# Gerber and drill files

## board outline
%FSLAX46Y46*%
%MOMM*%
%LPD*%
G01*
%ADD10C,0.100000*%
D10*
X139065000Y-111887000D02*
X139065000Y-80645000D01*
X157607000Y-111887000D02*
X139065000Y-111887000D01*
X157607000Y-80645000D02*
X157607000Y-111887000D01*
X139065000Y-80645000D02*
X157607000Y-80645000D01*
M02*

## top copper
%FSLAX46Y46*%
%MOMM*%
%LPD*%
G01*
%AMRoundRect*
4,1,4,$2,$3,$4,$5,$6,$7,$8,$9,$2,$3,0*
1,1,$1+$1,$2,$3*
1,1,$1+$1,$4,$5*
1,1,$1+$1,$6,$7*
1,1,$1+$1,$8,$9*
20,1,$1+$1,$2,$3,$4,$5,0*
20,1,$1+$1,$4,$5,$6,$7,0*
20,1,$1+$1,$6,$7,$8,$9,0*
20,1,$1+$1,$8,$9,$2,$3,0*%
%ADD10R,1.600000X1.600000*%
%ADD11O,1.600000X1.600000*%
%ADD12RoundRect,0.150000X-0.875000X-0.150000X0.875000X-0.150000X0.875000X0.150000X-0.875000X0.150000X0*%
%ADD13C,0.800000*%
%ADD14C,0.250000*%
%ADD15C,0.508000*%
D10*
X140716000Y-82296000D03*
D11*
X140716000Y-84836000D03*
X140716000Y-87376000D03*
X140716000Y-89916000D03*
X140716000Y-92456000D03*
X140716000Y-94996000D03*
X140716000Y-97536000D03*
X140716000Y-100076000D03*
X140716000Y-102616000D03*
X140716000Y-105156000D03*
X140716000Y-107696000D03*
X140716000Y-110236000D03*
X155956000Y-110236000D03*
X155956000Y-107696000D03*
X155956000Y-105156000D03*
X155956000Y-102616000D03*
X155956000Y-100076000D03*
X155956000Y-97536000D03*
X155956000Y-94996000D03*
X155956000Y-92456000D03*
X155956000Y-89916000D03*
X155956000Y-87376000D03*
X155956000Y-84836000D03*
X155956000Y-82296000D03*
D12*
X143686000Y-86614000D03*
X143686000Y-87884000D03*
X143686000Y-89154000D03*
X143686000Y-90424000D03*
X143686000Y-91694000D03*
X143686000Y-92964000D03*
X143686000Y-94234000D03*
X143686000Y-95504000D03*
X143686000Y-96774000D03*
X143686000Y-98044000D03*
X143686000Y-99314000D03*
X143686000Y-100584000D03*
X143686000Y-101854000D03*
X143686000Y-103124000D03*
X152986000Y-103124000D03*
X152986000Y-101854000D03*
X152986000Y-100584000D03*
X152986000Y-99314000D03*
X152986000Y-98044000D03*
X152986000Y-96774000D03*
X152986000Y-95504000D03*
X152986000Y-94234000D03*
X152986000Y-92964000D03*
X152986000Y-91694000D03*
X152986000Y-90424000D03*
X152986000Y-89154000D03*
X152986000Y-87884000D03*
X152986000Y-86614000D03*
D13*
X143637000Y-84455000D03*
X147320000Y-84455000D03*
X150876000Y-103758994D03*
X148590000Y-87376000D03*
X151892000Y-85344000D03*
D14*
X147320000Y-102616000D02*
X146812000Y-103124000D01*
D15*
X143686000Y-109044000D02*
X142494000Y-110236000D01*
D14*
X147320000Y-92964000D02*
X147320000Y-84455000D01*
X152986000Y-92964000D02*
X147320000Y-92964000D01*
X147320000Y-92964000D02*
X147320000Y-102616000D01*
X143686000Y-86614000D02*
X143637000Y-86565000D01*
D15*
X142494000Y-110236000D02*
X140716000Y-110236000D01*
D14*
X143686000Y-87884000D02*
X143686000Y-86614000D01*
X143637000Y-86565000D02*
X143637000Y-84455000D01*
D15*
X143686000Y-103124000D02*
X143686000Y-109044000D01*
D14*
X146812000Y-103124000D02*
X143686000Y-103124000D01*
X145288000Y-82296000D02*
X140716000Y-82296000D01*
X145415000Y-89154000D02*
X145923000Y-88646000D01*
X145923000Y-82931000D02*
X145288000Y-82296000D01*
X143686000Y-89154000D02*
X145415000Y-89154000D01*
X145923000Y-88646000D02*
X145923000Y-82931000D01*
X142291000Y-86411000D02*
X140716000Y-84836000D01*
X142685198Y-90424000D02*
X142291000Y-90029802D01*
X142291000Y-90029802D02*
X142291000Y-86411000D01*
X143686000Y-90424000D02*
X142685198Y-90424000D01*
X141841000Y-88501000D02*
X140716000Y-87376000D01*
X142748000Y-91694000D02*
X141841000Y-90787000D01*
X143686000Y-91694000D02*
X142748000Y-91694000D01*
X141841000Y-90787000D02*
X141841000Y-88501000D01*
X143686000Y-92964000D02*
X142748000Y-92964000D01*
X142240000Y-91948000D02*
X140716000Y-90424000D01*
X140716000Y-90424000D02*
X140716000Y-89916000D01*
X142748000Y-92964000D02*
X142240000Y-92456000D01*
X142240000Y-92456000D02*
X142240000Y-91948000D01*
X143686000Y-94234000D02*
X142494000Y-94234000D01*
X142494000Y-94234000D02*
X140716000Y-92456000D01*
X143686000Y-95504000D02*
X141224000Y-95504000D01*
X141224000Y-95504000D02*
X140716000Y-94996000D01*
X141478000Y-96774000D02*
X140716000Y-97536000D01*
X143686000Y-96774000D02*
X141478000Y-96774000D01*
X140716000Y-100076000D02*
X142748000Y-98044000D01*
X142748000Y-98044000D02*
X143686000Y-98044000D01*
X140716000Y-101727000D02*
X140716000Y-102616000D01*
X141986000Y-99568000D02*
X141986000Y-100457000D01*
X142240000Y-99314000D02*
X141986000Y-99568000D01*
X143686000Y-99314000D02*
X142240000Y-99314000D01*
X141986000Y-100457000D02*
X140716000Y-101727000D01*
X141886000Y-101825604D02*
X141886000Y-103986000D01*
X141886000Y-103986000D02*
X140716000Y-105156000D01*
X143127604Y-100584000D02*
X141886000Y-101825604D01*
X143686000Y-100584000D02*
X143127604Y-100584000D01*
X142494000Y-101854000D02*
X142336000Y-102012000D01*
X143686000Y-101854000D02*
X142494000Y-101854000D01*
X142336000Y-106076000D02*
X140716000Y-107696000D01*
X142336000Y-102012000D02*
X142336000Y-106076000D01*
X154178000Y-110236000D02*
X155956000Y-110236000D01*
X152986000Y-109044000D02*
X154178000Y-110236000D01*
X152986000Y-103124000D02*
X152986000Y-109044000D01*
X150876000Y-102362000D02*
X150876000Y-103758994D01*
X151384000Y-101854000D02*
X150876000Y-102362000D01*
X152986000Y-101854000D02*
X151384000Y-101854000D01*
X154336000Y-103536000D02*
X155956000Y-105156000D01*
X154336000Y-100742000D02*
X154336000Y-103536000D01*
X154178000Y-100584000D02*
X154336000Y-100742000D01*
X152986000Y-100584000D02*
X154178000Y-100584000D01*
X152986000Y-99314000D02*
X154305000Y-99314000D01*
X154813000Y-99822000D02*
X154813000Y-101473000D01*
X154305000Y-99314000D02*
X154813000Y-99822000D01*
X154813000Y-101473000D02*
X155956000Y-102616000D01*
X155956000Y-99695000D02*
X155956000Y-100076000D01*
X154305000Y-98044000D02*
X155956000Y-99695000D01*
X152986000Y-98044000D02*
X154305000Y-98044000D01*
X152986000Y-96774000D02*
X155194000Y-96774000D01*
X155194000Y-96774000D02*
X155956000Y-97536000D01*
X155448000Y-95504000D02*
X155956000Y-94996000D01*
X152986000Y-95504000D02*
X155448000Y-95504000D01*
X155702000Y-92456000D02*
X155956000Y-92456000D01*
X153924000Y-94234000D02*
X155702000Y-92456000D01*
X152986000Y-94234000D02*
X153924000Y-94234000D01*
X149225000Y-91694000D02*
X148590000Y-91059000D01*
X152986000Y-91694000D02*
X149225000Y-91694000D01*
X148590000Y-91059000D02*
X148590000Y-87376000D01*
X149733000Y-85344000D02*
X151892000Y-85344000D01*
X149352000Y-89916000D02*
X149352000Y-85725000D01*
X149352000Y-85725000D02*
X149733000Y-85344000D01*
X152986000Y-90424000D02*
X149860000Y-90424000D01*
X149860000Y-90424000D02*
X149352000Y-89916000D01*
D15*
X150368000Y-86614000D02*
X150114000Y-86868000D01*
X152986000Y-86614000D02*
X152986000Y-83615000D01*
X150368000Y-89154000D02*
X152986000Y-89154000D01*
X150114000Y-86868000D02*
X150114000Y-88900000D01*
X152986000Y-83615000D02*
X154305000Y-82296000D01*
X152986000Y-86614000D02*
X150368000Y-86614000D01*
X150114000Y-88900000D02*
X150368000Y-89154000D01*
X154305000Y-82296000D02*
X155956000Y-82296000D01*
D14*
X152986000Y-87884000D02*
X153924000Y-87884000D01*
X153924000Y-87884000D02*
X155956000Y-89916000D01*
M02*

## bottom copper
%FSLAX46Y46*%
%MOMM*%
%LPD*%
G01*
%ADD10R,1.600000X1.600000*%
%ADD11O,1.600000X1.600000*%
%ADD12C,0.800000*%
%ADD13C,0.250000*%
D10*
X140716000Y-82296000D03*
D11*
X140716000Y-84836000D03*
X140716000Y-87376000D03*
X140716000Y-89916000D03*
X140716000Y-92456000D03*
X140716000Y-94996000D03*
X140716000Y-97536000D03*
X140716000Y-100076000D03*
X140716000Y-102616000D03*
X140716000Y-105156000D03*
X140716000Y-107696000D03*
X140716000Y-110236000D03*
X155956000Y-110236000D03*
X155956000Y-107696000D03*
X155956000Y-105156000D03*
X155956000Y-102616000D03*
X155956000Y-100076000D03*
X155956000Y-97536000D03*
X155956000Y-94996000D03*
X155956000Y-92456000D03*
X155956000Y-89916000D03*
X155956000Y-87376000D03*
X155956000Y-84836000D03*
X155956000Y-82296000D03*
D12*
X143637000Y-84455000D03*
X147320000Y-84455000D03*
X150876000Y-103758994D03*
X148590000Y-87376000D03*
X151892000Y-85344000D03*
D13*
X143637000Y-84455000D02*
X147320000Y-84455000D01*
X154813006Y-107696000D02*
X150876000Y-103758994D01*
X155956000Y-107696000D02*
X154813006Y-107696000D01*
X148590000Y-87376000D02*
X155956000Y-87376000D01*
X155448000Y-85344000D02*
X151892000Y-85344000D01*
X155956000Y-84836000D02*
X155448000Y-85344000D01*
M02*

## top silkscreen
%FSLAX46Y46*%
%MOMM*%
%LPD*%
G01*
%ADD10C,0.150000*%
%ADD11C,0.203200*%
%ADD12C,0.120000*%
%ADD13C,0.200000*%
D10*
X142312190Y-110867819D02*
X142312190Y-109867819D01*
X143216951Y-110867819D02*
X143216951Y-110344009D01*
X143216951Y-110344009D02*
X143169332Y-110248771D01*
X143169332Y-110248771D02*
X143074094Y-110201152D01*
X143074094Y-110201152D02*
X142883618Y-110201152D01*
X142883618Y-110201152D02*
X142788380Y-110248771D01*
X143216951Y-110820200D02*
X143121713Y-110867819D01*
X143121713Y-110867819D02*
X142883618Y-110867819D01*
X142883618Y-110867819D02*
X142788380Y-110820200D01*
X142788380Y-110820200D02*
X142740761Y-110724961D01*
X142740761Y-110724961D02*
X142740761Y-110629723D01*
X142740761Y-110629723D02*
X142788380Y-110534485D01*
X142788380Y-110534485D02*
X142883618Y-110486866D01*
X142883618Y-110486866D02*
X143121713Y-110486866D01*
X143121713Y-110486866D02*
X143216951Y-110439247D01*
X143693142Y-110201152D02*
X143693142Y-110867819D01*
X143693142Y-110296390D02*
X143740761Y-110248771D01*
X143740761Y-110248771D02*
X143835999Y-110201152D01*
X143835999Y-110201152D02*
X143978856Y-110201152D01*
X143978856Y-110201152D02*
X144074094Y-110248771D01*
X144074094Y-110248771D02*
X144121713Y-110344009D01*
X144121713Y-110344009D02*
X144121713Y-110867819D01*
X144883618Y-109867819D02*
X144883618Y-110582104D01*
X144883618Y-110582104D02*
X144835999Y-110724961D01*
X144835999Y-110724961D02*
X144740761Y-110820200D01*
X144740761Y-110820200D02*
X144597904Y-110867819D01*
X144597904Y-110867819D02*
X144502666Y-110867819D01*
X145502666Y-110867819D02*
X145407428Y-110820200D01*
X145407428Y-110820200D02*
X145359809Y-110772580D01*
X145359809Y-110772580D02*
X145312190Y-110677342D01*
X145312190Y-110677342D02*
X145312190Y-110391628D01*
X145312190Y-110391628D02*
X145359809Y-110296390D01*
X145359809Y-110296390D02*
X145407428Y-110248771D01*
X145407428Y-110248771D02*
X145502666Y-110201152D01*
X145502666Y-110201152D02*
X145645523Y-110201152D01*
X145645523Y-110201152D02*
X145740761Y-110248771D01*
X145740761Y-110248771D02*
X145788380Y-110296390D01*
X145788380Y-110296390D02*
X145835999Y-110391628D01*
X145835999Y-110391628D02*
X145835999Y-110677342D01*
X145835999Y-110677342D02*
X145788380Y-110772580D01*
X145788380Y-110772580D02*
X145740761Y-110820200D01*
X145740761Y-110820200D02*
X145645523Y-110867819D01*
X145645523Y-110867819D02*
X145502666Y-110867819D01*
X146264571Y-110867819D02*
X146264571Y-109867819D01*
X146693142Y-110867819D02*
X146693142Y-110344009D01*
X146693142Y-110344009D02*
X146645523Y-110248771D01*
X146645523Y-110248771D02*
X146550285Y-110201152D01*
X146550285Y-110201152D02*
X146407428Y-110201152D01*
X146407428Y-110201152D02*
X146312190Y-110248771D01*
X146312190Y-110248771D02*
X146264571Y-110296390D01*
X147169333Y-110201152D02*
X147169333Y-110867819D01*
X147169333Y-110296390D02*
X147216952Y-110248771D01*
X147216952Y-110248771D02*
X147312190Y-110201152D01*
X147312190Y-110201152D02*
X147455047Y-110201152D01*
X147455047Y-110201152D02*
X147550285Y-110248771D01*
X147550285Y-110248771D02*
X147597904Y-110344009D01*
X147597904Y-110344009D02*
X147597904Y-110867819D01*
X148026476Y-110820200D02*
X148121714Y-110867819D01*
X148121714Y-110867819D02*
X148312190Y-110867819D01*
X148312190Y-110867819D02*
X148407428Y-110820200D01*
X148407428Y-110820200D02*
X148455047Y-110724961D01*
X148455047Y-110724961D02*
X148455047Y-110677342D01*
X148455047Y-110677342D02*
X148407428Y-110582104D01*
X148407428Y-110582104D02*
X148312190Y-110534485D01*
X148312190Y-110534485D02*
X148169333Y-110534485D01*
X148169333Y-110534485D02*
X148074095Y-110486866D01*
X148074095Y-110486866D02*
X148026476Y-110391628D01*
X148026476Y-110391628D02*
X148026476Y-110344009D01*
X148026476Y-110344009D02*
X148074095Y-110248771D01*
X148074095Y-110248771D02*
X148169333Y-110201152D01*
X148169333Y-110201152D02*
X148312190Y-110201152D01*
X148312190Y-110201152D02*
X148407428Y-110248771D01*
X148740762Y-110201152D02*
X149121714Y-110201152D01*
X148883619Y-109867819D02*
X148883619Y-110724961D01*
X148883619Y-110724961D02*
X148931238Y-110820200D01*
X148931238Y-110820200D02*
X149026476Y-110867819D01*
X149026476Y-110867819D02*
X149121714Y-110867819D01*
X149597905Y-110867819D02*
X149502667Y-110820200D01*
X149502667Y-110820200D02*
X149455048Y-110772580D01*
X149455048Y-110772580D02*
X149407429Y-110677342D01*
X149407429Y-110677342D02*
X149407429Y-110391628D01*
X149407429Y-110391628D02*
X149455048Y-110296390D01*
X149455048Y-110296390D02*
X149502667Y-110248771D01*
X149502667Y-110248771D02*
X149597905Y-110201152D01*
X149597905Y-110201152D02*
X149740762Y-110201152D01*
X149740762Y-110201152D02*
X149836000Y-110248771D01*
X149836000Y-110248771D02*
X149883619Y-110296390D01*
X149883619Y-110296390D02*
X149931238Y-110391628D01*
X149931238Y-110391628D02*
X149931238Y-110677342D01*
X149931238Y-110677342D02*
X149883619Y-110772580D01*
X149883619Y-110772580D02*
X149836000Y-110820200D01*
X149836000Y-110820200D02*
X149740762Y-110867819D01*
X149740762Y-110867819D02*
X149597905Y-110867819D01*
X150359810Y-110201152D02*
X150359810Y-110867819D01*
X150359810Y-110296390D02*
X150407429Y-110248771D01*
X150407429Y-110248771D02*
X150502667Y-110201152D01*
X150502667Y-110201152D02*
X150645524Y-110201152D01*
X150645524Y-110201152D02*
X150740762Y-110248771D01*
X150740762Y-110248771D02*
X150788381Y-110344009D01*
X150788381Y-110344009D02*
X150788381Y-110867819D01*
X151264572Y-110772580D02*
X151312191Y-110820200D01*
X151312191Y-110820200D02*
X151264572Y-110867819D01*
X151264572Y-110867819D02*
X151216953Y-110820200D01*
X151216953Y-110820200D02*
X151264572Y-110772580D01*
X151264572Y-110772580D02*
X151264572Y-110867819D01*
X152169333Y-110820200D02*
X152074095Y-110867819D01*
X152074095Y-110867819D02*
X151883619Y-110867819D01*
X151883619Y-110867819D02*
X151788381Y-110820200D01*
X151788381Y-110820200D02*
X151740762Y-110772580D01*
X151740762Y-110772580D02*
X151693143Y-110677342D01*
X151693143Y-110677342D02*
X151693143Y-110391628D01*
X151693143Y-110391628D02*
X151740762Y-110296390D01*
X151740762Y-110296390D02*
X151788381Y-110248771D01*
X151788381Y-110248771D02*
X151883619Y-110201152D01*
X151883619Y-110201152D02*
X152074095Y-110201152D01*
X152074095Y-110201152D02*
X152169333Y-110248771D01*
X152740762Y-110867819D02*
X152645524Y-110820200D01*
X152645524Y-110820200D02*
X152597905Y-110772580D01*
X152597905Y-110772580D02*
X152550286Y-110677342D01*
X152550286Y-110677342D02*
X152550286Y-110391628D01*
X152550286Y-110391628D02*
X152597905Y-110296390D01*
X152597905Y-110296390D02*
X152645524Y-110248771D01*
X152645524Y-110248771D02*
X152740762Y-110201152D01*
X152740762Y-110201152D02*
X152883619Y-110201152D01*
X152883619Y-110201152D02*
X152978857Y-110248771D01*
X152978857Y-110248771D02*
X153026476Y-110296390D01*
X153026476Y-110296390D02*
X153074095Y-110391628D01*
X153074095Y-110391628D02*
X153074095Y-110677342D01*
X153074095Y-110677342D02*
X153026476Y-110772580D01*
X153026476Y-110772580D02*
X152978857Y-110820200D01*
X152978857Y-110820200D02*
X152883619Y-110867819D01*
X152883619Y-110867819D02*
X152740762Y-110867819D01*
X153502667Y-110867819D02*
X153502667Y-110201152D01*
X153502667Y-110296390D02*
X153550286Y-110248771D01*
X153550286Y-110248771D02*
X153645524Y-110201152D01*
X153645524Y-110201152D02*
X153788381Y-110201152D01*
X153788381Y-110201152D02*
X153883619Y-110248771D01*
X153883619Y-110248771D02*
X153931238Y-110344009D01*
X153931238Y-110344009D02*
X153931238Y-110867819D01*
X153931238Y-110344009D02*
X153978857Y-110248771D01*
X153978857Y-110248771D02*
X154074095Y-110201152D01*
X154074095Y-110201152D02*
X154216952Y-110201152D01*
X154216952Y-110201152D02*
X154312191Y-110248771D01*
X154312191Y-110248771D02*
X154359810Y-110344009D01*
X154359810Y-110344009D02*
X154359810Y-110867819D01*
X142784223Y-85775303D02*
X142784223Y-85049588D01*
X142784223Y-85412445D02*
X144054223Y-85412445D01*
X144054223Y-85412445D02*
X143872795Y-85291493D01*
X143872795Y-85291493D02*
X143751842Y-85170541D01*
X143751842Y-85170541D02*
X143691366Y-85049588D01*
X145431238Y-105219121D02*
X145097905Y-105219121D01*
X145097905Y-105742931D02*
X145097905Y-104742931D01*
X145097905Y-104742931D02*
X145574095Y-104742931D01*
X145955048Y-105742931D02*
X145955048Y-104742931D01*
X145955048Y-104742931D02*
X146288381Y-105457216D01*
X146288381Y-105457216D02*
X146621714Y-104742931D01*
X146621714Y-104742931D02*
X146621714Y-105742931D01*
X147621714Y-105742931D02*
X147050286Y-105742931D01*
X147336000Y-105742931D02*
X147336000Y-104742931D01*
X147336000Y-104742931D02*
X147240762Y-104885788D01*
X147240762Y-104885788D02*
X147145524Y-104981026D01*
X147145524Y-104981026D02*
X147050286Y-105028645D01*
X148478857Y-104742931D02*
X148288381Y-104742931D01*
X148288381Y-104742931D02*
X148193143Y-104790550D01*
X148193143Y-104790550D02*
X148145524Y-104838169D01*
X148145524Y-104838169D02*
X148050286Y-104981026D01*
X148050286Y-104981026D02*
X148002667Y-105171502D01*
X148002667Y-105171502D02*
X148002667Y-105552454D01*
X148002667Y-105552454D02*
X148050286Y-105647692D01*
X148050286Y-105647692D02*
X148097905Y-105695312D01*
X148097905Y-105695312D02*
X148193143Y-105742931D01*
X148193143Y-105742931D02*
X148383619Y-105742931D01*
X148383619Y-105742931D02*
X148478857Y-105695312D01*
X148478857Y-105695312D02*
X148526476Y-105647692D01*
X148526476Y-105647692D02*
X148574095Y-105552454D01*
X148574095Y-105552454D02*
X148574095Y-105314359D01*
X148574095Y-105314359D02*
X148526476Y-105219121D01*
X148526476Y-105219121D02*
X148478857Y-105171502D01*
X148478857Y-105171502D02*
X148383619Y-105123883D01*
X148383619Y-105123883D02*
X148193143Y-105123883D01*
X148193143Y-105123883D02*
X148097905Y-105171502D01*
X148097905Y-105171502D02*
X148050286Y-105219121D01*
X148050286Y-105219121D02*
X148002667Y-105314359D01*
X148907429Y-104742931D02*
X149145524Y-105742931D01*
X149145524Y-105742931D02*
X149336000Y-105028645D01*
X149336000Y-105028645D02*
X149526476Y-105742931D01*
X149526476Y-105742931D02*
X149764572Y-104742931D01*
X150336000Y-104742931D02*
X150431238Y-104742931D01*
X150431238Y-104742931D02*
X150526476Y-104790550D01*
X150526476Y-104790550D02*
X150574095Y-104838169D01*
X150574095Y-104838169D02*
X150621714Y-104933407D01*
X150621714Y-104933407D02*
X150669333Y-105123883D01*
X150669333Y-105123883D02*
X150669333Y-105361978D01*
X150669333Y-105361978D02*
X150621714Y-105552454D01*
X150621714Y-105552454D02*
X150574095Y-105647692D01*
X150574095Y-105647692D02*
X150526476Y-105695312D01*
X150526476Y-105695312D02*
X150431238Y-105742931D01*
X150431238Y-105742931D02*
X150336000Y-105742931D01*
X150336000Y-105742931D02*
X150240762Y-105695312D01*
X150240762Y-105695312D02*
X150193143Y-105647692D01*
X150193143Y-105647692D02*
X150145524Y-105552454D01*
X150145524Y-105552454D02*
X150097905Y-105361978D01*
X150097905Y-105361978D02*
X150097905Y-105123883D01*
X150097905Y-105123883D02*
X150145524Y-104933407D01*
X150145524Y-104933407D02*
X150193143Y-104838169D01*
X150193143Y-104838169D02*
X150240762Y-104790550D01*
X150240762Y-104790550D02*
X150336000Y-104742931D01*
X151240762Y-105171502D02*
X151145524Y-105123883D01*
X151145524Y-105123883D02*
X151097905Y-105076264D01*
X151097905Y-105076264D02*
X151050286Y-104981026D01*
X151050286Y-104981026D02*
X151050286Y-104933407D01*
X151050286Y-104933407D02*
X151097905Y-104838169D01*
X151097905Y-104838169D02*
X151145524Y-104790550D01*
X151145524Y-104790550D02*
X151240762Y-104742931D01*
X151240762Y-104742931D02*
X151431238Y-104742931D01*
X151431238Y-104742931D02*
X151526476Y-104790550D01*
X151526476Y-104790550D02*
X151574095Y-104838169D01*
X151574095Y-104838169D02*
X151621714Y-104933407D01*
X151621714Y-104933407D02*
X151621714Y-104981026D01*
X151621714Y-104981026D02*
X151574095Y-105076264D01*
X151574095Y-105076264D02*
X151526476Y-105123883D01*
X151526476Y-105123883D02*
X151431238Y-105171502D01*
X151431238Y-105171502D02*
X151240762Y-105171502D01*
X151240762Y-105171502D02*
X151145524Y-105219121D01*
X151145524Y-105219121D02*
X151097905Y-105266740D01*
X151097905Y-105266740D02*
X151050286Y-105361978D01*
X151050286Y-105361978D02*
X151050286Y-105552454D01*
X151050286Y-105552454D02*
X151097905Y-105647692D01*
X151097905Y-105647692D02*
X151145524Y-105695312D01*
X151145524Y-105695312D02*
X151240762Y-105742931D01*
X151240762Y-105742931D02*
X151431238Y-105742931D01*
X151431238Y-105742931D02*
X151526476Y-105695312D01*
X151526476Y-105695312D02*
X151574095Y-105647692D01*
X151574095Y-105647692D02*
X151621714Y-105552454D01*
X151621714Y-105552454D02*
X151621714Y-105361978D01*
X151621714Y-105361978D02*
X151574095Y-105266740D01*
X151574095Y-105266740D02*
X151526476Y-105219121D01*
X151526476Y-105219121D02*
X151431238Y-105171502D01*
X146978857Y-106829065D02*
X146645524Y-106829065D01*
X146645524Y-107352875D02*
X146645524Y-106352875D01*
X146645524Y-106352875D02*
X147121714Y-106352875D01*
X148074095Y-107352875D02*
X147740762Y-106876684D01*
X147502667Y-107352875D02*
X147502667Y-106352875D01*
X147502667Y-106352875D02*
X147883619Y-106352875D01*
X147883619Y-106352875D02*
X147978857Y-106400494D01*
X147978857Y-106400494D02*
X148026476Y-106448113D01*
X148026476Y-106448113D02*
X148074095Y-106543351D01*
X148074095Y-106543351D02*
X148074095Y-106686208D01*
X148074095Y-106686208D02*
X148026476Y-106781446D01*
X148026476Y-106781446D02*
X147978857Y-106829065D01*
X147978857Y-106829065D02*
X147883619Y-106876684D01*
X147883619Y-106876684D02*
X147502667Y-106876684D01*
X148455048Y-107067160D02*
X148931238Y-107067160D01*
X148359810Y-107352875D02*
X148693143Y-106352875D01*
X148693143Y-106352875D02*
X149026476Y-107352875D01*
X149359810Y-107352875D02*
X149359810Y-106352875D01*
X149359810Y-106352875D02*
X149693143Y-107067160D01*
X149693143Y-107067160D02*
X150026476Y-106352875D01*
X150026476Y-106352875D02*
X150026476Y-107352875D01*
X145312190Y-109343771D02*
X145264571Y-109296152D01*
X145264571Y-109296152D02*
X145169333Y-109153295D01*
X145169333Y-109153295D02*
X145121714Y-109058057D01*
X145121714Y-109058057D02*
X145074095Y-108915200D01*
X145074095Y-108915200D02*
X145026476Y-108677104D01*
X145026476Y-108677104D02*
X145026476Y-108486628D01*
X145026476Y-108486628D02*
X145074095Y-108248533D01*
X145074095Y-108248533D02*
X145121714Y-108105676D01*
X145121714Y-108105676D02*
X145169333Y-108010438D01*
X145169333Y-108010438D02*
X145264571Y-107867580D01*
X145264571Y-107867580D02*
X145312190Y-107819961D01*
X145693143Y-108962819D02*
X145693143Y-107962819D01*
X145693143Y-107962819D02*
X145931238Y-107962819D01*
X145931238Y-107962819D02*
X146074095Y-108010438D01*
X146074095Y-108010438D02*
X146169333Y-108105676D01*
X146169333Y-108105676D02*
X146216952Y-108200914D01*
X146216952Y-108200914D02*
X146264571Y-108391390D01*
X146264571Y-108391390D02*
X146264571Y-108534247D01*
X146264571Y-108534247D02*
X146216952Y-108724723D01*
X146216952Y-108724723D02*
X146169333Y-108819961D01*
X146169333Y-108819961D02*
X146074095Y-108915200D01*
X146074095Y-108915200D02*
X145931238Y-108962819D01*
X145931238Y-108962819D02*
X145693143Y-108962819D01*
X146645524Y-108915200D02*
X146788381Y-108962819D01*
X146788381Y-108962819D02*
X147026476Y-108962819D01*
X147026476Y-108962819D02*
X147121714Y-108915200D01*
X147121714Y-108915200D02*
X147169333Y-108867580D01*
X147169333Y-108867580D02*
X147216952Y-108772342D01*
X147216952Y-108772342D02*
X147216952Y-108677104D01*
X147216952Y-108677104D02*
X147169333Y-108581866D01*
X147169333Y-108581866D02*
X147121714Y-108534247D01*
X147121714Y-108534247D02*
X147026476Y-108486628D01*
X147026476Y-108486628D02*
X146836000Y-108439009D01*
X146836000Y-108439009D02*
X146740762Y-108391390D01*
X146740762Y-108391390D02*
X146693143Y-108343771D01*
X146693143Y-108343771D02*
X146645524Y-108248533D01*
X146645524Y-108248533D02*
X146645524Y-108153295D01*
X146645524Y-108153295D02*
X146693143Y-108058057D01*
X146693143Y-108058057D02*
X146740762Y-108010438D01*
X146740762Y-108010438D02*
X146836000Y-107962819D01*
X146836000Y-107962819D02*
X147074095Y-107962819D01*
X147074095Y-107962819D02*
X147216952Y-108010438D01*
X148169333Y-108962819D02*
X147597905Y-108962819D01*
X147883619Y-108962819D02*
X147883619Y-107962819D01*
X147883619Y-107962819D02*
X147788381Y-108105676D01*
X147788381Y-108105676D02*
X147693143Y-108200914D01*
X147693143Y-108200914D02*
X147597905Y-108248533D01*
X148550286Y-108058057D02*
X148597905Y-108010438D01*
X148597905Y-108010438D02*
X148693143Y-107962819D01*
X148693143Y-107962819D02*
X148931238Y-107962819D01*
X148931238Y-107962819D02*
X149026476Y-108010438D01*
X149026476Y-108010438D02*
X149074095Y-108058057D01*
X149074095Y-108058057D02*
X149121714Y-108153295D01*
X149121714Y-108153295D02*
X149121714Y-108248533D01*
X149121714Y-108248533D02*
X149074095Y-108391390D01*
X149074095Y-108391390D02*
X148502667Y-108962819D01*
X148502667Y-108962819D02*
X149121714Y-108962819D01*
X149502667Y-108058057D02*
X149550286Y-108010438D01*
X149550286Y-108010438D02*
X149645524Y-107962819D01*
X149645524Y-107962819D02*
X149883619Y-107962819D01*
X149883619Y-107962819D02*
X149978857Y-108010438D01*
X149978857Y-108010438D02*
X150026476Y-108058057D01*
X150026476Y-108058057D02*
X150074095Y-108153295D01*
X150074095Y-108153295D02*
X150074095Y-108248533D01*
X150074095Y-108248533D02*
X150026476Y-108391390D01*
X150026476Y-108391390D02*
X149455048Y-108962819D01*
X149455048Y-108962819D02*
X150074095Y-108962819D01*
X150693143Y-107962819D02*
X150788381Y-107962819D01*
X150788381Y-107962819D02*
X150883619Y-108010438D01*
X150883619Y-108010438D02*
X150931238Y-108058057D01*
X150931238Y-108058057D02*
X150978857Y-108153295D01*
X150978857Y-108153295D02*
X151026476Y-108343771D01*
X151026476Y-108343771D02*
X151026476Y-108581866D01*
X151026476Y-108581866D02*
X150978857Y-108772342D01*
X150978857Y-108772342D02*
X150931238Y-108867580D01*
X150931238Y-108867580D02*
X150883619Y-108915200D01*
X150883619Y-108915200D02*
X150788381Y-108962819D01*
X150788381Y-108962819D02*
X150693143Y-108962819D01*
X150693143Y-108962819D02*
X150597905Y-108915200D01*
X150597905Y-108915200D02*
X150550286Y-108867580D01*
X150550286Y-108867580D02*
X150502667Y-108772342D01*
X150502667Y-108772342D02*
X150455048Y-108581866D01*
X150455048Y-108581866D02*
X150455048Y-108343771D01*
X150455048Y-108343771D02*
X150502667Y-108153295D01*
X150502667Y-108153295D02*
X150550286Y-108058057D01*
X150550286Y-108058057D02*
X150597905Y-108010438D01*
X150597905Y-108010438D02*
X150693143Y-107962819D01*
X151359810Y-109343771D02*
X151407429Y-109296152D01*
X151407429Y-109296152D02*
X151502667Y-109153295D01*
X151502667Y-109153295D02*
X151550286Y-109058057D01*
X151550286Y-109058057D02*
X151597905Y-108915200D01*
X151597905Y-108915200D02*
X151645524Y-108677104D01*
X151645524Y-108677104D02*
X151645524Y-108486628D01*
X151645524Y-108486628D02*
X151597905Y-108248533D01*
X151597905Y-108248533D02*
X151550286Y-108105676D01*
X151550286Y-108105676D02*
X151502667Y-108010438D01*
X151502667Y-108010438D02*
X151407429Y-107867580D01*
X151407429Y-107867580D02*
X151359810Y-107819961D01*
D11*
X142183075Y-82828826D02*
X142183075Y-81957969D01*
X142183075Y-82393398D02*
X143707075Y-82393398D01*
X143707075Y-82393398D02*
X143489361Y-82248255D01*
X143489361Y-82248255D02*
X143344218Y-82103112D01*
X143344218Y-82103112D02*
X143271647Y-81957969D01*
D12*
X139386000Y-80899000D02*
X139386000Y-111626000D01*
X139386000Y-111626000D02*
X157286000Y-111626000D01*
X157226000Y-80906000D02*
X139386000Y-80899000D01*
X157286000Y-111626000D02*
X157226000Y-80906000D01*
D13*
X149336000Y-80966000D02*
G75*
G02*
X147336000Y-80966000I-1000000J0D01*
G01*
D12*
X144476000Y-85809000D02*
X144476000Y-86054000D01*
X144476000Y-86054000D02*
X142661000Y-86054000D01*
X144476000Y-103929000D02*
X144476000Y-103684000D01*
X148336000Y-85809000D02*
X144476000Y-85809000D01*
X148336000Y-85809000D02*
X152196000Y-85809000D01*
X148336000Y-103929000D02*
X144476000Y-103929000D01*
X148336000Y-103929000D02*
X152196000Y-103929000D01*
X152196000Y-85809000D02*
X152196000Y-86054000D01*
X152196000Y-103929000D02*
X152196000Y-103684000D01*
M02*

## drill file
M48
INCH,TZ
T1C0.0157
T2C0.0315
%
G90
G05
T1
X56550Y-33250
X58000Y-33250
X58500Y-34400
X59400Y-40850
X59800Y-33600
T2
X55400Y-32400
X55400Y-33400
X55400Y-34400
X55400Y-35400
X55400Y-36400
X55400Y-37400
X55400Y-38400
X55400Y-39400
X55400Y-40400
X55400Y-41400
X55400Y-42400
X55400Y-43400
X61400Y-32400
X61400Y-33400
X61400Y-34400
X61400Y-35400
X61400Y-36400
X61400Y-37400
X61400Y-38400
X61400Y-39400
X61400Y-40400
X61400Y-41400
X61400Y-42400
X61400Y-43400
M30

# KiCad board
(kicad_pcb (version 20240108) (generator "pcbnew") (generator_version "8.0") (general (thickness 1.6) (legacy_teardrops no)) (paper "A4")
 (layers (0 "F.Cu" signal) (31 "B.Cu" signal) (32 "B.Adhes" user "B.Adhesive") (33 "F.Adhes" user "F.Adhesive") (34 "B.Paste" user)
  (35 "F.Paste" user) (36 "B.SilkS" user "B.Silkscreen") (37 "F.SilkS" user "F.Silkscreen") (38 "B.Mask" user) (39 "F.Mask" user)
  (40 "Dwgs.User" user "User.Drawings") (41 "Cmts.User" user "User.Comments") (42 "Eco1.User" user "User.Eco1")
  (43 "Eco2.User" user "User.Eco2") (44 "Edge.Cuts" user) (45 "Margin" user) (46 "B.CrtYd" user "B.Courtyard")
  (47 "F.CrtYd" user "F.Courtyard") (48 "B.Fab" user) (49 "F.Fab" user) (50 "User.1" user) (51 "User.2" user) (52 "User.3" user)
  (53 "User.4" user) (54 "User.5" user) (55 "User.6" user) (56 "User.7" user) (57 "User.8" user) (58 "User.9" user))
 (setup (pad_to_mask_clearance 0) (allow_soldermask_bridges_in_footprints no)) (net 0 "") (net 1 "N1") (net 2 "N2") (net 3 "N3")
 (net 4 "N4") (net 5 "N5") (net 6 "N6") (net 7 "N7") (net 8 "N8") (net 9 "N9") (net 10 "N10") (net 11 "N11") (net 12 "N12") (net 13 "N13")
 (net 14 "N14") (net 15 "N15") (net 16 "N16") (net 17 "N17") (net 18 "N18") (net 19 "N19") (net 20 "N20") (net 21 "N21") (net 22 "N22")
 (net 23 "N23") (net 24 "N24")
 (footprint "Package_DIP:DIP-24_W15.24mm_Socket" (layer "F.Cu") (at 140.716 82.296)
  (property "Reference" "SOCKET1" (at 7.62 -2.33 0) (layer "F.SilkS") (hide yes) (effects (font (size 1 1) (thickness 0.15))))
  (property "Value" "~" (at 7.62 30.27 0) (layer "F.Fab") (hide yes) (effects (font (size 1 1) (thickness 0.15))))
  (fp_line (start -1.33 -1.397) (end -1.33 29.33) (stroke (width 0.12) (type solid)) (layer "F.SilkS"))
  (fp_line (start -1.33 29.33) (end 16.57 29.33) (stroke (width 0.12) (type solid)) (layer "F.SilkS"))
  (fp_line (start 16.51 -1.39) (end -1.33 -1.397) (stroke (width 0.12) (type solid)) (layer "F.SilkS"))
  (fp_line (start 16.57 29.33) (end 16.51 -1.39) (stroke (width 0.12) (type solid)) (layer "F.SilkS"))
  (fp_arc (start 8.62 -1.33) (mid 7.62 -0.33) (end 6.62 -1.33) (stroke (width 0.2) (type solid)) (layer "F.SilkS"))
  (pad "1" thru_hole rect (at 0 0) (size 1.6 1.6) (drill 0.8) (layers "*.Cu" "*.Mask") (remove_unused_layers no) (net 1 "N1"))
  (pad "2" thru_hole oval (at 0 2.54) (size 1.6 1.6) (drill 0.8) (layers "*.Cu" "*.Mask") (remove_unused_layers no) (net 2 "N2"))
  (pad "3" thru_hole oval (at 0 5.08) (size 1.6 1.6) (drill 0.8) (layers "*.Cu" "*.Mask") (remove_unused_layers no) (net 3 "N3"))
  (pad "4" thru_hole oval (at 0 7.62) (size 1.6 1.6) (drill 0.8) (layers "*.Cu" "*.Mask") (remove_unused_layers no) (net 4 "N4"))
  (pad "5" thru_hole oval (at 0 10.16) (size 1.6 1.6) (drill 0.8) (layers "*.Cu" "*.Mask") (remove_unused_layers no) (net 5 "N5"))
  (pad "6" thru_hole oval (at 0 12.7) (size 1.6 1.6) (drill 0.8) (layers "*.Cu" "*.Mask") (remove_unused_layers no) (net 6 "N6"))
  (pad "7" thru_hole oval (at 0 15.24) (size 1.6 1.6) (drill 0.8) (layers "*.Cu" "*.Mask") (remove_unused_layers no) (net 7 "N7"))
  (pad "8" thru_hole oval (at 0 17.78) (size 1.6 1.6) (drill 0.8) (layers "*.Cu" "*.Mask") (remove_unused_layers no) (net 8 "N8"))
  (pad "9" thru_hole oval (at 0 20.32) (size 1.6 1.6) (drill 0.8) (layers "*.Cu" "*.Mask") (remove_unused_layers no) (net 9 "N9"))
  (pad "10" thru_hole oval (at 0 22.86) (size 1.6 1.6) (drill 0.8) (layers "*.Cu" "*.Mask") (remove_unused_layers no) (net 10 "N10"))
  (pad "11" thru_hole oval (at 0 25.4) (size 1.6 1.6) (drill 0.8) (layers "*.Cu" "*.Mask") (remove_unused_layers no) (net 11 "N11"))
  (pad "12" thru_hole oval (at 0 27.94) (size 1.6 1.6) (drill 0.8) (layers "*.Cu" "*.Mask") (remove_unused_layers no) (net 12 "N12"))
  (pad "13" thru_hole oval (at 15.24 27.94) (size 1.6 1.6) (drill 0.8) (layers "*.Cu" "*.Mask") (remove_unused_layers no) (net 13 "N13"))
  (pad "14" thru_hole oval (at 15.24 25.4) (size 1.6 1.6) (drill 0.8) (layers "*.Cu" "*.Mask") (remove_unused_layers no) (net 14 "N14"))
  (pad "15" thru_hole oval (at 15.24 22.86) (size 1.6 1.6) (drill 0.8) (layers "*.Cu" "*.Mask") (remove_unused_layers no) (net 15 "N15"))
  (pad "16" thru_hole oval (at 15.24 20.32) (size 1.6 1.6) (drill 0.8) (layers "*.Cu" "*.Mask") (remove_unused_layers no) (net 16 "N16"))
  (pad "17" thru_hole oval (at 15.24 17.78) (size 1.6 1.6) (drill 0.8) (layers "*.Cu" "*.Mask") (remove_unused_layers no) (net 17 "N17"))
  (pad "18" thru_hole oval (at 15.24 15.24) (size 1.6 1.6) (drill 0.8) (layers "*.Cu" "*.Mask") (remove_unused_layers no) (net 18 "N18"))
  (pad "19" thru_hole oval (at 15.24 12.7) (size 1.6 1.6) (drill 0.8) (layers "*.Cu" "*.Mask") (remove_unused_layers no) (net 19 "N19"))
  (pad "20" thru_hole oval (at 15.24 10.16) (size 1.6 1.6) (drill 0.8) (layers "*.Cu" "*.Mask") (remove_unused_layers no) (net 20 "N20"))
  (pad "21" thru_hole oval (at 15.24 7.62) (size 1.6 1.6) (drill 0.8) (layers "*.Cu" "*.Mask") (remove_unused_layers no) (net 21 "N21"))
  (pad "22" thru_hole oval (at 15.24 5.08) (size 1.6 1.6) (drill 0.8) (layers "*.Cu" "*.Mask") (remove_unused_layers no) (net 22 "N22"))
  (pad "23" thru_hole oval (at 15.24 2.54) (size 1.6 1.6) (drill 0.8) (layers "*.Cu" "*.Mask") (remove_unused_layers no) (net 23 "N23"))
  (pad "24" thru_hole oval (at 15.24 0) (size 1.6 1.6) (drill 0.8) (layers "*.Cu" "*.Mask") (remove_unused_layers no) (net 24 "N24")))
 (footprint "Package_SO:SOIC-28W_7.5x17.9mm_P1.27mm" (layer "F.Cu") (at 148.336 94.869)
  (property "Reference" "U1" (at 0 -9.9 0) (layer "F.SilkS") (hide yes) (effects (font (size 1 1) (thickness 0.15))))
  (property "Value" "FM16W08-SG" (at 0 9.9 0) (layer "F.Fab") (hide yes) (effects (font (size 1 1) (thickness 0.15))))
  (fp_line (start -3.86 -9.06) (end -3.86 -8.815) (stroke (width 0.12) (type solid)) (layer "F.SilkS"))
  (fp_line (start -3.86 -8.815) (end -5.675 -8.815) (stroke (width 0.12) (type solid)) (layer "F.SilkS"))
  (fp_line (start -3.86 9.06) (end -3.86 8.815) (stroke (width 0.12) (type solid)) (layer "F.SilkS"))
  (fp_line (start 0 -9.06) (end -3.86 -9.06) (stroke (width 0.12) (type solid)) (layer "F.SilkS"))
  (fp_line (start 0 -9.06) (end 3.86 -9.06) (stroke (width 0.12) (type solid)) (layer "F.SilkS"))
  (fp_line (start 0 9.06) (end -3.86 9.06) (stroke (width 0.12) (type solid)) (layer "F.SilkS"))
  (fp_line (start 0 9.06) (end 3.86 9.06) (stroke (width 0.12) (type solid)) (layer "F.SilkS"))
  (fp_line (start 3.86 -9.06) (end 3.86 -8.815) (stroke (width 0.12) (type solid)) (layer "F.SilkS"))
  (fp_line (start 3.86 9.06) (end 3.86 8.815) (stroke (width 0.12) (type solid)) (layer "F.SilkS"))
  (pad "1" smd roundrect (at -4.65 -8.255) (size 2.05 0.6) (layers "F.Cu" "F.Paste" "F.Mask") (roundrect_rratio 0.25) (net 12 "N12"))
  (pad "2" smd roundrect (at -4.65 -6.985) (size 2.05 0.6) (layers "F.Cu" "F.Paste" "F.Mask") (roundrect_rratio 0.25) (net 12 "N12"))
  (pad "3" smd roundrect (at -4.65 -5.715) (size 2.05 0.6) (layers "F.Cu" "F.Paste" "F.Mask") (roundrect_rratio 0.25) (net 1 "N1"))
  (pad "4" smd roundrect (at -4.65 -4.445) (size 2.05 0.6) (layers "F.Cu" "F.Paste" "F.Mask") (roundrect_rratio 0.25) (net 2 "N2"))
  (pad "5" smd roundrect (at -4.65 -3.175) (size 2.05 0.6) (layers "F.Cu" "F.Paste" "F.Mask") (roundrect_rratio 0.25) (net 3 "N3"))
  (pad "6" smd roundrect (at -4.65 -1.905) (size 2.05 0.6) (layers "F.Cu" "F.Paste" "F.Mask") (roundrect_rratio 0.25) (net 4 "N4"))
  (pad "7" smd roundrect (at -4.65 -0.635) (size 2.05 0.6) (layers "F.Cu" "F.Paste" "F.Mask") (roundrect_rratio 0.25) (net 5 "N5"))
  (pad "8" smd roundrect (at -4.65 0.635) (size 2.05 0.6) (layers "F.Cu" "F.Paste" "F.Mask") (roundrect_rratio 0.25) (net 6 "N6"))
  (pad "9" smd roundrect (at -4.65 1.905) (size 2.05 0.6) (layers "F.Cu" "F.Paste" "F.Mask") (roundrect_rratio 0.25) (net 7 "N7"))
  (pad "10" smd roundrect (at -4.65 3.175) (size 2.05 0.6) (layers "F.Cu" "F.Paste" "F.Mask") (roundrect_rratio 0.25) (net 8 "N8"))
  (pad "11" smd roundrect (at -4.65 4.445) (size 2.05 0.6) (layers "F.Cu" "F.Paste" "F.Mask") (roundrect_rratio 0.25) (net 9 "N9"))
  (pad "12" smd roundrect (at -4.65 5.715) (size 2.05 0.6) (layers "F.Cu" "F.Paste" "F.Mask") (roundrect_rratio 0.25) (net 10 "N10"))
  (pad "13" smd roundrect (at -4.65 6.985) (size 2.05 0.6) (layers "F.Cu" "F.Paste" "F.Mask") (roundrect_rratio 0.25) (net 11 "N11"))
  (pad "14" smd roundrect (at -4.65 8.255) (size 2.05 0.6) (layers "F.Cu" "F.Paste" "F.Mask") (roundrect_rratio 0.25) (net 12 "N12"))
  (pad "15" smd roundrect (at 4.65 8.255) (size 2.05 0.6) (layers "F.Cu" "F.Paste" "F.Mask") (roundrect_rratio 0.25) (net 13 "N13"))
  (pad "16" smd roundrect (at 4.65 6.985) (size 2.05 0.6) (layers "F.Cu" "F.Paste" "F.Mask") (roundrect_rratio 0.25) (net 14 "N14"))
  (pad "17" smd roundrect (at 4.65 5.715) (size 2.05 0.6) (layers "F.Cu" "F.Paste" "F.Mask") (roundrect_rratio 0.25) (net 15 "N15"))
  (pad "18" smd roundrect (at 4.65 4.445) (size 2.05 0.6) (layers "F.Cu" "F.Paste" "F.Mask") (roundrect_rratio 0.25) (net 16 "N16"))
  (pad "19" smd roundrect (at 4.65 3.175) (size 2.05 0.6) (layers "F.Cu" "F.Paste" "F.Mask") (roundrect_rratio 0.25) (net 17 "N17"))
  (pad "20" smd roundrect (at 4.65 1.905) (size 2.05 0.6) (layers "F.Cu" "F.Paste" "F.Mask") (roundrect_rratio 0.25) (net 18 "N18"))
  (pad "21" smd roundrect (at 4.65 0.635) (size 2.05 0.6) (layers "F.Cu" "F.Paste" "F.Mask") (roundrect_rratio 0.25) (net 19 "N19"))
  (pad "22" smd roundrect (at 4.65 -0.635) (size 2.05 0.6) (layers "F.Cu" "F.Paste" "F.Mask") (roundrect_rratio 0.25) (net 20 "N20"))
  (pad "23" smd roundrect (at 4.65 -1.905) (size 2.05 0.6) (layers "F.Cu" "F.Paste" "F.Mask") (roundrect_rratio 0.25) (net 12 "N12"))
  (pad "24" smd roundrect (at 4.65 -3.175) (size 2.05 0.6) (layers "F.Cu" "F.Paste" "F.Mask") (roundrect_rratio 0.25) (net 22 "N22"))
  (pad "25" smd roundrect (at 4.65 -4.445) (size 2.05 0.6) (layers "F.Cu" "F.Paste" "F.Mask") (roundrect_rratio 0.25) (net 23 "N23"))
  (pad "26" smd roundrect (at 4.65 -5.715) (size 2.05 0.6) (layers "F.Cu" "F.Paste" "F.Mask") (roundrect_rratio 0.25) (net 24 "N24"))
  (pad "27" smd roundrect (at 4.65 -6.985) (size 2.05 0.6) (layers "F.Cu" "F.Paste" "F.Mask") (roundrect_rratio 0.25) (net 21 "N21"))
  (pad "28" smd roundrect (at 4.65 -8.255) (size 2.05 0.6) (layers "F.Cu" "F.Paste" "F.Mask") (roundrect_rratio 0.25) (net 24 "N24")))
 (gr_line (start 139.065 80.645) (end 157.607 80.645) (stroke (width 0.1) (type default)) (layer "Edge.Cuts"))
 (gr_line (start 157.607 111.887) (end 139.065 111.887) (stroke (width 0.1) (type default)) (layer "Edge.Cuts"))
 (gr_line (start 157.607 80.645) (end 157.607 111.887) (stroke (width 0.1) (type default)) (layer "Edge.Cuts"))
 (gr_line (start 139.065 111.887) (end 139.065 80.645) (stroke (width 0.1) (type default)) (layer "Edge.Cuts"))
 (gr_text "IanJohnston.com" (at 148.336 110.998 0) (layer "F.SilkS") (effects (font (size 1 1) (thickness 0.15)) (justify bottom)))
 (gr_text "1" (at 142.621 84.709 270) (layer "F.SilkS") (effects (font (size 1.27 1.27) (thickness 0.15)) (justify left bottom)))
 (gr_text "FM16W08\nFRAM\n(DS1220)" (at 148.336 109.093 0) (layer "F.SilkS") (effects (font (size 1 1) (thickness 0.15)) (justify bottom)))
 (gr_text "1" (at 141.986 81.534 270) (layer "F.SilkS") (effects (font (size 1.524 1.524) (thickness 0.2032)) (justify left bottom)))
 (segment (start 147.32 102.616) (end 146.812 103.124) (width 0.25) (layer "F.Cu") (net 12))
 (segment (start 143.686 109.044) (end 142.494 110.236) (width 0.508) (layer "F.Cu") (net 12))
 (segment (start 147.32 92.964) (end 147.32 84.455) (width 0.25) (layer "F.Cu") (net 12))
 (segment (start 152.986 92.964) (end 147.32 92.964) (width 0.25) (layer "F.Cu") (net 12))
 (segment (start 147.32 92.964) (end 147.32 102.616) (width 0.25) (layer "F.Cu") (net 12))
 (segment (start 143.686 86.614) (end 143.637 86.565) (width 0.25) (layer "F.Cu") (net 12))
 (segment (start 142.494 110.236) (end 140.716 110.236) (width 0.508) (layer "F.Cu") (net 12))
 (segment (start 143.686 87.884) (end 143.686 86.614) (width 0.25) (layer "F.Cu") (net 12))
 (segment (start 143.637 86.565) (end 143.637 84.455) (width 0.25) (layer "F.Cu") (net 12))
 (segment (start 143.686 103.124) (end 143.686 109.044) (width 0.508) (layer "F.Cu") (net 12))
 (segment (start 146.812 103.124) (end 143.686 103.124) (width 0.25) (layer "F.Cu") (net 12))
 (via (at 143.637 84.455) (size 0.8) (drill 0.4) (layers "F.Cu" "B.Cu") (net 12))
 (via (at 147.32 84.455) (size 0.8) (drill 0.4) (layers "F.Cu" "B.Cu") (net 12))
 (segment (start 143.637 84.455) (end 147.32 84.455) (width 0.25) (layer "B.Cu") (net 12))
 (segment (start 145.288 82.296) (end 140.716 82.296) (width 0.25) (layer "F.Cu") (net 1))
 (segment (start 145.415 89.154) (end 145.923 88.646) (width 0.25) (layer "F.Cu") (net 1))
 (segment (start 145.923 82.931) (end 145.288 82.296) (width 0.25) (layer "F.Cu") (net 1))
 (segment (start 143.686 89.154) (end 145.415 89.154) (width 0.25) (layer "F.Cu") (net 1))
 (segment (start 145.923 88.646) (end 145.923 82.931) (width 0.25) (layer "F.Cu") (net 1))
 (segment (start 142.291 86.411) (end 140.716 84.836) (width 0.25) (layer "F.Cu") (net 2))
 (segment (start 142.685198 90.424) (end 142.291 90.029802) (width 0.25) (layer "F.Cu") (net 2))
 (segment (start 142.291 90.029802) (end 142.291 86.411) (width 0.25) (layer "F.Cu") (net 2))
 (segment (start 143.686 90.424) (end 142.685198 90.424) (width 0.25) (layer "F.Cu") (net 2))
 (segment (start 141.841 88.501) (end 140.716 87.376) (width 0.25) (layer "F.Cu") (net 3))
 (segment (start 142.748 91.694) (end 141.841 90.787) (width 0.25) (layer "F.Cu") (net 3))
 (segment (start 143.686 91.694) (end 142.748 91.694) (width 0.25) (layer "F.Cu") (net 3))
 (segment (start 141.841 90.787) (end 141.841 88.501) (width 0.25) (layer "F.Cu") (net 3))
 (segment (start 143.686 92.964) (end 142.748 92.964) (width 0.25) (layer "F.Cu") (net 4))
 (segment (start 142.24 91.948) (end 140.716 90.424) (width 0.25) (layer "F.Cu") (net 4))
 (segment (start 140.716 90.424) (end 140.716 89.916) (width 0.25) (layer "F.Cu") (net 4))
 (segment (start 142.748 92.964) (end 142.24 92.456) (width 0.25) (layer "F.Cu") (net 4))
 (segment (start 142.24 92.456) (end 142.24 91.948) (width 0.25) (layer "F.Cu") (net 4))
 (segment (start 143.686 94.234) (end 142.494 94.234) (width 0.25) (layer "F.Cu") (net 5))
 (segment (start 142.494 94.234) (end 140.716 92.456) (width 0.25) (layer "F.Cu") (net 5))
 (segment (start 143.686 95.504) (end 141.224 95.504) (width 0.25) (layer "F.Cu") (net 6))
 (segment (start 141.224 95.504) (end 140.716 94.996) (width 0.25) (layer "F.Cu") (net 6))
 (segment (start 141.478 96.774) (end 140.716 97.536) (width 0.25) (layer "F.Cu") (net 7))
 (segment (start 143.686 96.774) (end 141.478 96.774) (width 0.25) (layer "F.Cu") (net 7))
 (segment (start 140.716 100.076) (end 142.748 98.044) (width 0.25) (layer "F.Cu") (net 8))
 (segment (start 142.748 98.044) (end 143.686 98.044) (width 0.25) (layer "F.Cu") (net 8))
 (segment (start 140.716 101.727) (end 140.716 102.616) (width 0.25) (layer "F.Cu") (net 9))
 (segment (start 141.986 99.568) (end 141.986 100.457) (width 0.25) (layer "F.Cu") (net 9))
 (segment (start 142.24 99.314) (end 141.986 99.568) (width 0.25) (layer "F.Cu") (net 9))
 (segment (start 143.686 99.314) (end 142.24 99.314) (width 0.25) (layer "F.Cu") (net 9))
 (segment (start 141.986 100.457) (end 140.716 101.727) (width 0.25) (layer "F.Cu") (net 9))
 (segment (start 141.886 101.825604) (end 141.886 103.986) (width 0.25) (layer "F.Cu") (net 10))
 (segment (start 141.886 103.986) (end 140.716 105.156) (width 0.25) (layer "F.Cu") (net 10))
 (segment (start 143.127604 100.584) (end 141.886 101.825604) (width 0.25) (layer "F.Cu") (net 10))
 (segment (start 143.686 100.584) (end 143.127604 100.584) (width 0.25) (layer "F.Cu") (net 10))
 (segment (start 142.494 101.854) (end 142.336 102.012) (width 0.25) (layer "F.Cu") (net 11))
 (segment (start 143.686 101.854) (end 142.494 101.854) (width 0.25) (layer "F.Cu") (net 11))
 (segment (start 142.336 106.076) (end 140.716 107.696) (width 0.25) (layer "F.Cu") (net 11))
 (segment (start 142.336 102.012) (end 142.336 106.076) (width 0.25) (layer "F.Cu") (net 11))
 (segment (start 154.178 110.236) (end 155.956 110.236) (width 0.25) (layer "F.Cu") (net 13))
 (segment (start 152.986 109.044) (end 154.178 110.236) (width 0.25) (layer "F.Cu") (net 13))
 (segment (start 152.986 103.124) (end 152.986 109.044) (width 0.25) (layer "F.Cu") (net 13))
 (segment (start 150.876 102.362) (end 150.876 103.758994) (width 0.25) (layer "F.Cu") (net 14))
 (segment (start 151.384 101.854) (end 150.876 102.362) (width 0.25) (layer "F.Cu") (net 14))
 (segment (start 152.986 101.854) (end 151.384 101.854) (width 0.25) (layer "F.Cu") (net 14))
 (via (at 150.876 103.758994) (size 0.8) (drill 0.4) (layers "F.Cu" "B.Cu") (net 14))
 (segment (start 154.813006 107.696) (end 150.876 103.758994) (width 0.25) (layer "B.Cu") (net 14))
 (segment (start 155.956 107.696) (end 154.813006 107.696) (width 0.25) (layer "B.Cu") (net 14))
 (segment (start 154.336 103.536) (end 155.956 105.156) (width 0.25) (layer "F.Cu") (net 15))
 (segment (start 154.336 100.742) (end 154.336 103.536) (width 0.25) (layer "F.Cu") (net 15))
 (segment (start 154.178 100.584) (end 154.336 100.742) (width 0.25) (layer "F.Cu") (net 15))
 (segment (start 152.986 100.584) (end 154.178 100.584) (width 0.25) (layer "F.Cu") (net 15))
 (segment (start 152.986 99.314) (end 154.305 99.314) (width 0.25) (layer "F.Cu") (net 16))
 (segment (start 154.813 99.822) (end 154.813 101.473) (width 0.25) (layer "F.Cu") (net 16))
 (segment (start 154.305 99.314) (end 154.813 99.822) (width 0.25) (layer "F.Cu") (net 16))
 (segment (start 154.813 101.473) (end 155.956 102.616) (width 0.25) (layer "F.Cu") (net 16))
 (segment (start 155.956 99.695) (end 155.956 100.076) (width 0.25) (layer "F.Cu") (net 17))
 (segment (start 154.305 98.044) (end 155.956 99.695) (width 0.25) (layer "F.Cu") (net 17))
 (segment (start 152.986 98.044) (end 154.305 98.044) (width 0.25) (layer "F.Cu") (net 17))
 (segment (start 152.986 96.774) (end 155.194 96.774) (width 0.25) (layer "F.Cu") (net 18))
 (segment (start 155.194 96.774) (end 155.956 97.536) (width 0.25) (layer "F.Cu") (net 18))
 (segment (start 155.448 95.504) (end 155.956 94.996) (width 0.25) (layer "F.Cu") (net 19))
 (segment (start 152.986 95.504) (end 155.448 95.504) (width 0.25) (layer "F.Cu") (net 19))
 (segment (start 155.702 92.456) (end 155.956 92.456) (width 0.25) (layer "F.Cu") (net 20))
 (segment (start 153.924 94.234) (end 155.702 92.456) (width 0.25) (layer "F.Cu") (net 20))
 (segment (start 152.986 94.234) (end 153.924 94.234) (width 0.25) (layer "F.Cu") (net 20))
 (segment (start 149.225 91.694) (end 148.59 91.059) (width 0.25) (layer "F.Cu") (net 22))
 (segment (start 152.986 91.694) (end 149.225 91.694) (width 0.25) (layer "F.Cu") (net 22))
 (segment (start 148.59 91.059) (end 148.59 87.376) (width 0.25) (layer "F.Cu") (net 22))
 (via (at 148.59 87.376) (size 0.8) (drill 0.4) (layers "F.Cu" "B.Cu") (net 22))
 (segment (start 148.59 87.376) (end 155.956 87.376) (width 0.25) (layer "B.Cu") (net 22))
 (segment (start 149.733 85.344) (end 151.892 85.344) (width 0.25) (layer "F.Cu") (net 23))
 (segment (start 149.352 89.916) (end 149.352 85.725) (width 0.25) (layer "F.Cu") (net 23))
 (segment (start 149.352 85.725) (end 149.733 85.344) (width 0.25) (layer "F.Cu") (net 23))
 (segment (start 152.986 90.424) (end 149.86 90.424) (width 0.25) (layer "F.Cu") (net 23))
 (segment (start 149.86 90.424) (end 149.352 89.916) (width 0.25) (layer "F.Cu") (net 23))
 (via (at 151.892 85.344) (size 0.8) (drill 0.4) (layers "F.Cu" "B.Cu") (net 23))
 (segment (start 155.448 85.344) (end 151.892 85.344) (width 0.25) (layer "B.Cu") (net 23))
 (segment (start 155.956 84.836) (end 155.448 85.344) (width 0.25) (layer "B.Cu") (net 23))
 (segment (start 150.368 86.614) (end 150.114 86.868) (width 0.508) (layer "F.Cu") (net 24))
 (segment (start 152.986 86.614) (end 152.986 83.615) (width 0.508) (layer "F.Cu") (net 24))
 (segment (start 150.368 89.154) (end 152.986 89.154) (width 0.508) (layer "F.Cu") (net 24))
 (segment (start 150.114 86.868) (end 150.114 88.9) (width 0.508) (layer "F.Cu") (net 24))
 (segment (start 152.986 83.615) (end 154.305 82.296) (width 0.508) (layer "F.Cu") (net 24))
 (segment (start 152.986 86.614) (end 150.368 86.614) (width 0.508) (layer "F.Cu") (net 24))
 (segment (start 150.114 88.9) (end 150.368 89.154) (width 0.508) (layer "F.Cu") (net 24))
 (segment (start 154.305 82.296) (end 155.956 82.296) (width 0.508) (layer "F.Cu") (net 24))
 (segment (start 152.986 87.884) (end 153.924 87.884) (width 0.25) (layer "F.Cu") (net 21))
 (segment (start 153.924 87.884) (end 155.956 89.916) (width 0.25) (layer "F.Cu") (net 21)))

